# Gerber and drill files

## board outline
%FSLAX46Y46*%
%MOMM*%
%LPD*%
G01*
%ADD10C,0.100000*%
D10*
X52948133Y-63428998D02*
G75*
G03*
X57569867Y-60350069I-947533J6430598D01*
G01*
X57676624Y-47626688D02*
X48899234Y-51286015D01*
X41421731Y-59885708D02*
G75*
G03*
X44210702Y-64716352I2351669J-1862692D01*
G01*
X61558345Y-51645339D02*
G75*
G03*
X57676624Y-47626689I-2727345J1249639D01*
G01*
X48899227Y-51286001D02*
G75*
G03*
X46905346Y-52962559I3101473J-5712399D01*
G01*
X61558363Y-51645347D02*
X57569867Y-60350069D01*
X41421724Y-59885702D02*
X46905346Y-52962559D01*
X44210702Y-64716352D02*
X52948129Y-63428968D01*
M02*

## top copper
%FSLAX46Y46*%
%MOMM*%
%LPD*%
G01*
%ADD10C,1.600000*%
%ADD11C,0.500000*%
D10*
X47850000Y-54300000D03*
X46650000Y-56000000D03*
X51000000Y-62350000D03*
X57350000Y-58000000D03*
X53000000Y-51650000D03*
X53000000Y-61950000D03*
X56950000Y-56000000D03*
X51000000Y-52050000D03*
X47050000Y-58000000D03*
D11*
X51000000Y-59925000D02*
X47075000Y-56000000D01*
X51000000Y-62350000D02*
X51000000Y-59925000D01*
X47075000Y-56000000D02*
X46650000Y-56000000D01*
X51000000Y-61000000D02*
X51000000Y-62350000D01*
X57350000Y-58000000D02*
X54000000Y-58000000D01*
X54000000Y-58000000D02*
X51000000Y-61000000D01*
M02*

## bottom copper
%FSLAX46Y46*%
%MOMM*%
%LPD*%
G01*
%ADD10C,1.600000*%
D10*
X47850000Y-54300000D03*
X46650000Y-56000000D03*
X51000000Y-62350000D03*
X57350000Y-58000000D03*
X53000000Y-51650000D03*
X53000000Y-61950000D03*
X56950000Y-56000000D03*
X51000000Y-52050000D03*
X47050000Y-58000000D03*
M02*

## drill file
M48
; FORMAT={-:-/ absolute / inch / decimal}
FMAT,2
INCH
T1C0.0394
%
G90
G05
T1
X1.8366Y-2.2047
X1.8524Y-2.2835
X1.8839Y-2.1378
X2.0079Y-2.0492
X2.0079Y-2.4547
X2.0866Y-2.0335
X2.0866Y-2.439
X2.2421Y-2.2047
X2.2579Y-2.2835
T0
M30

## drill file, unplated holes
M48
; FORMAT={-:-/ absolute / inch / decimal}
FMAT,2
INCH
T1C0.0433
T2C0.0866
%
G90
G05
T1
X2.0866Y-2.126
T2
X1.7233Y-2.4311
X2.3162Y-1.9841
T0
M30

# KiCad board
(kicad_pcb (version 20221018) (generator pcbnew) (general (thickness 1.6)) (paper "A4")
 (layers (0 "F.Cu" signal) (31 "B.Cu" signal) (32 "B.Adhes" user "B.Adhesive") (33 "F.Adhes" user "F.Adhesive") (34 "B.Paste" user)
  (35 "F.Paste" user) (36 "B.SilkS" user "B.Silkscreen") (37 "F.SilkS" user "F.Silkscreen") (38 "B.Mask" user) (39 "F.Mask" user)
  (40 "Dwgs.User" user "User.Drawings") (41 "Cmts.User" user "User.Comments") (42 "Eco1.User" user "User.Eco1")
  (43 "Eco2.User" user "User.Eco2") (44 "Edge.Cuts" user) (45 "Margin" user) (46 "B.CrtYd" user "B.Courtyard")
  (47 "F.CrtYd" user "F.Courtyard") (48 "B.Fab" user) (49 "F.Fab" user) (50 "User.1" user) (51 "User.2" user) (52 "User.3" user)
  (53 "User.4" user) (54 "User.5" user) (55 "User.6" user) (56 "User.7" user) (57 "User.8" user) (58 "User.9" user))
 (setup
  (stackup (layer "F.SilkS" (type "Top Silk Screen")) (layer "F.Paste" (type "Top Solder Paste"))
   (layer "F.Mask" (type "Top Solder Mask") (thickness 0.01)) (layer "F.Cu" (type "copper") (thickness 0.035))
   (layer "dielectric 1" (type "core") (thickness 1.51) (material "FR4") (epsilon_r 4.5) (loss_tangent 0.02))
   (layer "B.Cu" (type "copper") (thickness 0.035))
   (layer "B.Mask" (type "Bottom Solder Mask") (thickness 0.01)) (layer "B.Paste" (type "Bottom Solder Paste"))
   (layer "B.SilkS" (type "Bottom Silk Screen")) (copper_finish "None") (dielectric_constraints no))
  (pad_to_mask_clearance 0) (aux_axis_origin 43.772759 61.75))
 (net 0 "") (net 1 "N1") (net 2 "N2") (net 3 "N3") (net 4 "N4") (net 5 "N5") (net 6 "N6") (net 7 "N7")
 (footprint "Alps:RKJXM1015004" (layer "F.Cu") (at 52 57)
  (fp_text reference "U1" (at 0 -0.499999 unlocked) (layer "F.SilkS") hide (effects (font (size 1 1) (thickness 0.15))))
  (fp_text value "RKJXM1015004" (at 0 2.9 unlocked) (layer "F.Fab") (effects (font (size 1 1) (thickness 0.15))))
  (pad "" np_thru_hole circle (at 1 -3) (size 1.1 1.1) (drill 1.1) (layers "F&B.Cu" "*.Mask"))
  (pad "1" thru_hole circle (at -4.15 -2.7) (size 1.6 1.6) (drill 1) (layers "*.Cu" "*.Mask") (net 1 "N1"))
  (pad "2" thru_hole circle (at -5.35 -1) (size 1.6 1.6) (drill 1) (layers "*.Cu" "*.Mask") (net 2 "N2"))
  (pad "2" thru_hole circle (at -1 5.35) (size 1.6 1.6) (drill 1) (layers "*.Cu" "*.Mask") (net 2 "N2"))
  (pad "2" thru_hole circle (at 5.35 1) (size 1.6 1.6) (drill 1) (layers "*.Cu" "*.Mask") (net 2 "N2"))
  (pad "3" thru_hole circle (at 1 -5.35) (size 1.6 1.6) (drill 1) (layers "*.Cu" "*.Mask") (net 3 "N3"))
  (pad "4" thru_hole circle (at 1 4.95) (size 1.6 1.6) (drill 1) (layers "*.Cu" "*.Mask") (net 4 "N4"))
  (pad "5" thru_hole circle (at 4.95 -1) (size 1.6 1.6) (drill 1) (layers "*.Cu" "*.Mask") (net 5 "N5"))
  (pad "6" thru_hole circle (at -1 -4.95) (size 1.6 1.6) (drill 1) (layers "*.Cu" "*.Mask") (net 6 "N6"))
  (pad "7" thru_hole circle (at -4.95 1) (size 1.6 1.6) (drill 1) (layers "*.Cu" "*.Mask") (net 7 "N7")))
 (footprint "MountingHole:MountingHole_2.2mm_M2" (layer "F.Cu") (at 43.772759 61.75)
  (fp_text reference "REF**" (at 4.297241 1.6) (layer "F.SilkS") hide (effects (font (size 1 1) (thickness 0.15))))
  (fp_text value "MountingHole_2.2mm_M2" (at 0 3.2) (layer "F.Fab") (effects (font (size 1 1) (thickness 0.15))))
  (pad "" np_thru_hole circle (at 0 0) (size 2.2 2.2) (drill 2.2) (layers "*.Cu" "*.Mask")))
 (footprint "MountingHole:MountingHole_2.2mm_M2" (layer "F.Cu") (at 58.831 50.3957)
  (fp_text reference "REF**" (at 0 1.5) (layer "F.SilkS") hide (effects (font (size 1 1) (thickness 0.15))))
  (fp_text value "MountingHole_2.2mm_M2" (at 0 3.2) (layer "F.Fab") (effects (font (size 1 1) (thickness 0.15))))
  (pad "" np_thru_hole circle (at 0 0) (size 2.2 2.2) (drill 2.2) (layers "*.Cu" "*.Mask")))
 (gr_arc (start 57.569867 60.350069) (mid 55.60436 62.407942) (end 52.948129 63.428968) (stroke (width 0.1) (type solid))
  (layer "Edge.Cuts"))
 (gr_line (start 57.676624 47.626688) (end 48.899234 51.286015) (stroke (width 0.1) (type solid)) (layer "Edge.Cuts"))
 (gr_arc (start 44.210702 64.716352) (mid 41.175323 63.248395) (end 41.421724 59.885702) (stroke (width 0.1) (type solid))
  (layer "Edge.Cuts"))
 (gr_arc (start 57.676624 47.626688) (mid 60.988764 48.311458) (end 61.558363 51.645347) (stroke (width 0.1) (type solid))
  (layer "Edge.Cuts"))
 (gr_arc (start 46.905346 52.962559) (mid 47.817439 52.023375) (end 48.899234 51.286015) (stroke (width 0.1) (type solid))
  (layer "Edge.Cuts"))
 (gr_line (start 61.558363 51.645347) (end 57.569867 60.350069) (stroke (width 0.1) (type solid)) (layer "Edge.Cuts"))
 (gr_line (start 41.421724 59.885702) (end 46.905346 52.962559) (stroke (width 0.1) (type solid)) (layer "Edge.Cuts"))
 (gr_line (start 44.210702 64.716352) (end 52.948129 63.428968) (stroke (width 0.1) (type solid)) (layer "Edge.Cuts"))
 (segment (start 51 59.925) (end 47.075 56) (width 0.5) (layer "F.Cu") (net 2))
 (segment (start 51 62.35) (end 51 59.925) (width 0.5) (layer "F.Cu") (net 2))
 (segment (start 47.075 56) (end 46.65 56) (width 0.5) (layer "F.Cu") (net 2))
 (segment (start 51 61) (end 51 62.35) (width 0.5) (layer "F.Cu") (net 2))
 (segment (start 57.35 58) (end 54 58) (width 0.5) (layer "F.Cu") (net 2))
 (segment (start 54 58) (end 51 61) (width 0.5) (layer "F.Cu") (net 2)))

